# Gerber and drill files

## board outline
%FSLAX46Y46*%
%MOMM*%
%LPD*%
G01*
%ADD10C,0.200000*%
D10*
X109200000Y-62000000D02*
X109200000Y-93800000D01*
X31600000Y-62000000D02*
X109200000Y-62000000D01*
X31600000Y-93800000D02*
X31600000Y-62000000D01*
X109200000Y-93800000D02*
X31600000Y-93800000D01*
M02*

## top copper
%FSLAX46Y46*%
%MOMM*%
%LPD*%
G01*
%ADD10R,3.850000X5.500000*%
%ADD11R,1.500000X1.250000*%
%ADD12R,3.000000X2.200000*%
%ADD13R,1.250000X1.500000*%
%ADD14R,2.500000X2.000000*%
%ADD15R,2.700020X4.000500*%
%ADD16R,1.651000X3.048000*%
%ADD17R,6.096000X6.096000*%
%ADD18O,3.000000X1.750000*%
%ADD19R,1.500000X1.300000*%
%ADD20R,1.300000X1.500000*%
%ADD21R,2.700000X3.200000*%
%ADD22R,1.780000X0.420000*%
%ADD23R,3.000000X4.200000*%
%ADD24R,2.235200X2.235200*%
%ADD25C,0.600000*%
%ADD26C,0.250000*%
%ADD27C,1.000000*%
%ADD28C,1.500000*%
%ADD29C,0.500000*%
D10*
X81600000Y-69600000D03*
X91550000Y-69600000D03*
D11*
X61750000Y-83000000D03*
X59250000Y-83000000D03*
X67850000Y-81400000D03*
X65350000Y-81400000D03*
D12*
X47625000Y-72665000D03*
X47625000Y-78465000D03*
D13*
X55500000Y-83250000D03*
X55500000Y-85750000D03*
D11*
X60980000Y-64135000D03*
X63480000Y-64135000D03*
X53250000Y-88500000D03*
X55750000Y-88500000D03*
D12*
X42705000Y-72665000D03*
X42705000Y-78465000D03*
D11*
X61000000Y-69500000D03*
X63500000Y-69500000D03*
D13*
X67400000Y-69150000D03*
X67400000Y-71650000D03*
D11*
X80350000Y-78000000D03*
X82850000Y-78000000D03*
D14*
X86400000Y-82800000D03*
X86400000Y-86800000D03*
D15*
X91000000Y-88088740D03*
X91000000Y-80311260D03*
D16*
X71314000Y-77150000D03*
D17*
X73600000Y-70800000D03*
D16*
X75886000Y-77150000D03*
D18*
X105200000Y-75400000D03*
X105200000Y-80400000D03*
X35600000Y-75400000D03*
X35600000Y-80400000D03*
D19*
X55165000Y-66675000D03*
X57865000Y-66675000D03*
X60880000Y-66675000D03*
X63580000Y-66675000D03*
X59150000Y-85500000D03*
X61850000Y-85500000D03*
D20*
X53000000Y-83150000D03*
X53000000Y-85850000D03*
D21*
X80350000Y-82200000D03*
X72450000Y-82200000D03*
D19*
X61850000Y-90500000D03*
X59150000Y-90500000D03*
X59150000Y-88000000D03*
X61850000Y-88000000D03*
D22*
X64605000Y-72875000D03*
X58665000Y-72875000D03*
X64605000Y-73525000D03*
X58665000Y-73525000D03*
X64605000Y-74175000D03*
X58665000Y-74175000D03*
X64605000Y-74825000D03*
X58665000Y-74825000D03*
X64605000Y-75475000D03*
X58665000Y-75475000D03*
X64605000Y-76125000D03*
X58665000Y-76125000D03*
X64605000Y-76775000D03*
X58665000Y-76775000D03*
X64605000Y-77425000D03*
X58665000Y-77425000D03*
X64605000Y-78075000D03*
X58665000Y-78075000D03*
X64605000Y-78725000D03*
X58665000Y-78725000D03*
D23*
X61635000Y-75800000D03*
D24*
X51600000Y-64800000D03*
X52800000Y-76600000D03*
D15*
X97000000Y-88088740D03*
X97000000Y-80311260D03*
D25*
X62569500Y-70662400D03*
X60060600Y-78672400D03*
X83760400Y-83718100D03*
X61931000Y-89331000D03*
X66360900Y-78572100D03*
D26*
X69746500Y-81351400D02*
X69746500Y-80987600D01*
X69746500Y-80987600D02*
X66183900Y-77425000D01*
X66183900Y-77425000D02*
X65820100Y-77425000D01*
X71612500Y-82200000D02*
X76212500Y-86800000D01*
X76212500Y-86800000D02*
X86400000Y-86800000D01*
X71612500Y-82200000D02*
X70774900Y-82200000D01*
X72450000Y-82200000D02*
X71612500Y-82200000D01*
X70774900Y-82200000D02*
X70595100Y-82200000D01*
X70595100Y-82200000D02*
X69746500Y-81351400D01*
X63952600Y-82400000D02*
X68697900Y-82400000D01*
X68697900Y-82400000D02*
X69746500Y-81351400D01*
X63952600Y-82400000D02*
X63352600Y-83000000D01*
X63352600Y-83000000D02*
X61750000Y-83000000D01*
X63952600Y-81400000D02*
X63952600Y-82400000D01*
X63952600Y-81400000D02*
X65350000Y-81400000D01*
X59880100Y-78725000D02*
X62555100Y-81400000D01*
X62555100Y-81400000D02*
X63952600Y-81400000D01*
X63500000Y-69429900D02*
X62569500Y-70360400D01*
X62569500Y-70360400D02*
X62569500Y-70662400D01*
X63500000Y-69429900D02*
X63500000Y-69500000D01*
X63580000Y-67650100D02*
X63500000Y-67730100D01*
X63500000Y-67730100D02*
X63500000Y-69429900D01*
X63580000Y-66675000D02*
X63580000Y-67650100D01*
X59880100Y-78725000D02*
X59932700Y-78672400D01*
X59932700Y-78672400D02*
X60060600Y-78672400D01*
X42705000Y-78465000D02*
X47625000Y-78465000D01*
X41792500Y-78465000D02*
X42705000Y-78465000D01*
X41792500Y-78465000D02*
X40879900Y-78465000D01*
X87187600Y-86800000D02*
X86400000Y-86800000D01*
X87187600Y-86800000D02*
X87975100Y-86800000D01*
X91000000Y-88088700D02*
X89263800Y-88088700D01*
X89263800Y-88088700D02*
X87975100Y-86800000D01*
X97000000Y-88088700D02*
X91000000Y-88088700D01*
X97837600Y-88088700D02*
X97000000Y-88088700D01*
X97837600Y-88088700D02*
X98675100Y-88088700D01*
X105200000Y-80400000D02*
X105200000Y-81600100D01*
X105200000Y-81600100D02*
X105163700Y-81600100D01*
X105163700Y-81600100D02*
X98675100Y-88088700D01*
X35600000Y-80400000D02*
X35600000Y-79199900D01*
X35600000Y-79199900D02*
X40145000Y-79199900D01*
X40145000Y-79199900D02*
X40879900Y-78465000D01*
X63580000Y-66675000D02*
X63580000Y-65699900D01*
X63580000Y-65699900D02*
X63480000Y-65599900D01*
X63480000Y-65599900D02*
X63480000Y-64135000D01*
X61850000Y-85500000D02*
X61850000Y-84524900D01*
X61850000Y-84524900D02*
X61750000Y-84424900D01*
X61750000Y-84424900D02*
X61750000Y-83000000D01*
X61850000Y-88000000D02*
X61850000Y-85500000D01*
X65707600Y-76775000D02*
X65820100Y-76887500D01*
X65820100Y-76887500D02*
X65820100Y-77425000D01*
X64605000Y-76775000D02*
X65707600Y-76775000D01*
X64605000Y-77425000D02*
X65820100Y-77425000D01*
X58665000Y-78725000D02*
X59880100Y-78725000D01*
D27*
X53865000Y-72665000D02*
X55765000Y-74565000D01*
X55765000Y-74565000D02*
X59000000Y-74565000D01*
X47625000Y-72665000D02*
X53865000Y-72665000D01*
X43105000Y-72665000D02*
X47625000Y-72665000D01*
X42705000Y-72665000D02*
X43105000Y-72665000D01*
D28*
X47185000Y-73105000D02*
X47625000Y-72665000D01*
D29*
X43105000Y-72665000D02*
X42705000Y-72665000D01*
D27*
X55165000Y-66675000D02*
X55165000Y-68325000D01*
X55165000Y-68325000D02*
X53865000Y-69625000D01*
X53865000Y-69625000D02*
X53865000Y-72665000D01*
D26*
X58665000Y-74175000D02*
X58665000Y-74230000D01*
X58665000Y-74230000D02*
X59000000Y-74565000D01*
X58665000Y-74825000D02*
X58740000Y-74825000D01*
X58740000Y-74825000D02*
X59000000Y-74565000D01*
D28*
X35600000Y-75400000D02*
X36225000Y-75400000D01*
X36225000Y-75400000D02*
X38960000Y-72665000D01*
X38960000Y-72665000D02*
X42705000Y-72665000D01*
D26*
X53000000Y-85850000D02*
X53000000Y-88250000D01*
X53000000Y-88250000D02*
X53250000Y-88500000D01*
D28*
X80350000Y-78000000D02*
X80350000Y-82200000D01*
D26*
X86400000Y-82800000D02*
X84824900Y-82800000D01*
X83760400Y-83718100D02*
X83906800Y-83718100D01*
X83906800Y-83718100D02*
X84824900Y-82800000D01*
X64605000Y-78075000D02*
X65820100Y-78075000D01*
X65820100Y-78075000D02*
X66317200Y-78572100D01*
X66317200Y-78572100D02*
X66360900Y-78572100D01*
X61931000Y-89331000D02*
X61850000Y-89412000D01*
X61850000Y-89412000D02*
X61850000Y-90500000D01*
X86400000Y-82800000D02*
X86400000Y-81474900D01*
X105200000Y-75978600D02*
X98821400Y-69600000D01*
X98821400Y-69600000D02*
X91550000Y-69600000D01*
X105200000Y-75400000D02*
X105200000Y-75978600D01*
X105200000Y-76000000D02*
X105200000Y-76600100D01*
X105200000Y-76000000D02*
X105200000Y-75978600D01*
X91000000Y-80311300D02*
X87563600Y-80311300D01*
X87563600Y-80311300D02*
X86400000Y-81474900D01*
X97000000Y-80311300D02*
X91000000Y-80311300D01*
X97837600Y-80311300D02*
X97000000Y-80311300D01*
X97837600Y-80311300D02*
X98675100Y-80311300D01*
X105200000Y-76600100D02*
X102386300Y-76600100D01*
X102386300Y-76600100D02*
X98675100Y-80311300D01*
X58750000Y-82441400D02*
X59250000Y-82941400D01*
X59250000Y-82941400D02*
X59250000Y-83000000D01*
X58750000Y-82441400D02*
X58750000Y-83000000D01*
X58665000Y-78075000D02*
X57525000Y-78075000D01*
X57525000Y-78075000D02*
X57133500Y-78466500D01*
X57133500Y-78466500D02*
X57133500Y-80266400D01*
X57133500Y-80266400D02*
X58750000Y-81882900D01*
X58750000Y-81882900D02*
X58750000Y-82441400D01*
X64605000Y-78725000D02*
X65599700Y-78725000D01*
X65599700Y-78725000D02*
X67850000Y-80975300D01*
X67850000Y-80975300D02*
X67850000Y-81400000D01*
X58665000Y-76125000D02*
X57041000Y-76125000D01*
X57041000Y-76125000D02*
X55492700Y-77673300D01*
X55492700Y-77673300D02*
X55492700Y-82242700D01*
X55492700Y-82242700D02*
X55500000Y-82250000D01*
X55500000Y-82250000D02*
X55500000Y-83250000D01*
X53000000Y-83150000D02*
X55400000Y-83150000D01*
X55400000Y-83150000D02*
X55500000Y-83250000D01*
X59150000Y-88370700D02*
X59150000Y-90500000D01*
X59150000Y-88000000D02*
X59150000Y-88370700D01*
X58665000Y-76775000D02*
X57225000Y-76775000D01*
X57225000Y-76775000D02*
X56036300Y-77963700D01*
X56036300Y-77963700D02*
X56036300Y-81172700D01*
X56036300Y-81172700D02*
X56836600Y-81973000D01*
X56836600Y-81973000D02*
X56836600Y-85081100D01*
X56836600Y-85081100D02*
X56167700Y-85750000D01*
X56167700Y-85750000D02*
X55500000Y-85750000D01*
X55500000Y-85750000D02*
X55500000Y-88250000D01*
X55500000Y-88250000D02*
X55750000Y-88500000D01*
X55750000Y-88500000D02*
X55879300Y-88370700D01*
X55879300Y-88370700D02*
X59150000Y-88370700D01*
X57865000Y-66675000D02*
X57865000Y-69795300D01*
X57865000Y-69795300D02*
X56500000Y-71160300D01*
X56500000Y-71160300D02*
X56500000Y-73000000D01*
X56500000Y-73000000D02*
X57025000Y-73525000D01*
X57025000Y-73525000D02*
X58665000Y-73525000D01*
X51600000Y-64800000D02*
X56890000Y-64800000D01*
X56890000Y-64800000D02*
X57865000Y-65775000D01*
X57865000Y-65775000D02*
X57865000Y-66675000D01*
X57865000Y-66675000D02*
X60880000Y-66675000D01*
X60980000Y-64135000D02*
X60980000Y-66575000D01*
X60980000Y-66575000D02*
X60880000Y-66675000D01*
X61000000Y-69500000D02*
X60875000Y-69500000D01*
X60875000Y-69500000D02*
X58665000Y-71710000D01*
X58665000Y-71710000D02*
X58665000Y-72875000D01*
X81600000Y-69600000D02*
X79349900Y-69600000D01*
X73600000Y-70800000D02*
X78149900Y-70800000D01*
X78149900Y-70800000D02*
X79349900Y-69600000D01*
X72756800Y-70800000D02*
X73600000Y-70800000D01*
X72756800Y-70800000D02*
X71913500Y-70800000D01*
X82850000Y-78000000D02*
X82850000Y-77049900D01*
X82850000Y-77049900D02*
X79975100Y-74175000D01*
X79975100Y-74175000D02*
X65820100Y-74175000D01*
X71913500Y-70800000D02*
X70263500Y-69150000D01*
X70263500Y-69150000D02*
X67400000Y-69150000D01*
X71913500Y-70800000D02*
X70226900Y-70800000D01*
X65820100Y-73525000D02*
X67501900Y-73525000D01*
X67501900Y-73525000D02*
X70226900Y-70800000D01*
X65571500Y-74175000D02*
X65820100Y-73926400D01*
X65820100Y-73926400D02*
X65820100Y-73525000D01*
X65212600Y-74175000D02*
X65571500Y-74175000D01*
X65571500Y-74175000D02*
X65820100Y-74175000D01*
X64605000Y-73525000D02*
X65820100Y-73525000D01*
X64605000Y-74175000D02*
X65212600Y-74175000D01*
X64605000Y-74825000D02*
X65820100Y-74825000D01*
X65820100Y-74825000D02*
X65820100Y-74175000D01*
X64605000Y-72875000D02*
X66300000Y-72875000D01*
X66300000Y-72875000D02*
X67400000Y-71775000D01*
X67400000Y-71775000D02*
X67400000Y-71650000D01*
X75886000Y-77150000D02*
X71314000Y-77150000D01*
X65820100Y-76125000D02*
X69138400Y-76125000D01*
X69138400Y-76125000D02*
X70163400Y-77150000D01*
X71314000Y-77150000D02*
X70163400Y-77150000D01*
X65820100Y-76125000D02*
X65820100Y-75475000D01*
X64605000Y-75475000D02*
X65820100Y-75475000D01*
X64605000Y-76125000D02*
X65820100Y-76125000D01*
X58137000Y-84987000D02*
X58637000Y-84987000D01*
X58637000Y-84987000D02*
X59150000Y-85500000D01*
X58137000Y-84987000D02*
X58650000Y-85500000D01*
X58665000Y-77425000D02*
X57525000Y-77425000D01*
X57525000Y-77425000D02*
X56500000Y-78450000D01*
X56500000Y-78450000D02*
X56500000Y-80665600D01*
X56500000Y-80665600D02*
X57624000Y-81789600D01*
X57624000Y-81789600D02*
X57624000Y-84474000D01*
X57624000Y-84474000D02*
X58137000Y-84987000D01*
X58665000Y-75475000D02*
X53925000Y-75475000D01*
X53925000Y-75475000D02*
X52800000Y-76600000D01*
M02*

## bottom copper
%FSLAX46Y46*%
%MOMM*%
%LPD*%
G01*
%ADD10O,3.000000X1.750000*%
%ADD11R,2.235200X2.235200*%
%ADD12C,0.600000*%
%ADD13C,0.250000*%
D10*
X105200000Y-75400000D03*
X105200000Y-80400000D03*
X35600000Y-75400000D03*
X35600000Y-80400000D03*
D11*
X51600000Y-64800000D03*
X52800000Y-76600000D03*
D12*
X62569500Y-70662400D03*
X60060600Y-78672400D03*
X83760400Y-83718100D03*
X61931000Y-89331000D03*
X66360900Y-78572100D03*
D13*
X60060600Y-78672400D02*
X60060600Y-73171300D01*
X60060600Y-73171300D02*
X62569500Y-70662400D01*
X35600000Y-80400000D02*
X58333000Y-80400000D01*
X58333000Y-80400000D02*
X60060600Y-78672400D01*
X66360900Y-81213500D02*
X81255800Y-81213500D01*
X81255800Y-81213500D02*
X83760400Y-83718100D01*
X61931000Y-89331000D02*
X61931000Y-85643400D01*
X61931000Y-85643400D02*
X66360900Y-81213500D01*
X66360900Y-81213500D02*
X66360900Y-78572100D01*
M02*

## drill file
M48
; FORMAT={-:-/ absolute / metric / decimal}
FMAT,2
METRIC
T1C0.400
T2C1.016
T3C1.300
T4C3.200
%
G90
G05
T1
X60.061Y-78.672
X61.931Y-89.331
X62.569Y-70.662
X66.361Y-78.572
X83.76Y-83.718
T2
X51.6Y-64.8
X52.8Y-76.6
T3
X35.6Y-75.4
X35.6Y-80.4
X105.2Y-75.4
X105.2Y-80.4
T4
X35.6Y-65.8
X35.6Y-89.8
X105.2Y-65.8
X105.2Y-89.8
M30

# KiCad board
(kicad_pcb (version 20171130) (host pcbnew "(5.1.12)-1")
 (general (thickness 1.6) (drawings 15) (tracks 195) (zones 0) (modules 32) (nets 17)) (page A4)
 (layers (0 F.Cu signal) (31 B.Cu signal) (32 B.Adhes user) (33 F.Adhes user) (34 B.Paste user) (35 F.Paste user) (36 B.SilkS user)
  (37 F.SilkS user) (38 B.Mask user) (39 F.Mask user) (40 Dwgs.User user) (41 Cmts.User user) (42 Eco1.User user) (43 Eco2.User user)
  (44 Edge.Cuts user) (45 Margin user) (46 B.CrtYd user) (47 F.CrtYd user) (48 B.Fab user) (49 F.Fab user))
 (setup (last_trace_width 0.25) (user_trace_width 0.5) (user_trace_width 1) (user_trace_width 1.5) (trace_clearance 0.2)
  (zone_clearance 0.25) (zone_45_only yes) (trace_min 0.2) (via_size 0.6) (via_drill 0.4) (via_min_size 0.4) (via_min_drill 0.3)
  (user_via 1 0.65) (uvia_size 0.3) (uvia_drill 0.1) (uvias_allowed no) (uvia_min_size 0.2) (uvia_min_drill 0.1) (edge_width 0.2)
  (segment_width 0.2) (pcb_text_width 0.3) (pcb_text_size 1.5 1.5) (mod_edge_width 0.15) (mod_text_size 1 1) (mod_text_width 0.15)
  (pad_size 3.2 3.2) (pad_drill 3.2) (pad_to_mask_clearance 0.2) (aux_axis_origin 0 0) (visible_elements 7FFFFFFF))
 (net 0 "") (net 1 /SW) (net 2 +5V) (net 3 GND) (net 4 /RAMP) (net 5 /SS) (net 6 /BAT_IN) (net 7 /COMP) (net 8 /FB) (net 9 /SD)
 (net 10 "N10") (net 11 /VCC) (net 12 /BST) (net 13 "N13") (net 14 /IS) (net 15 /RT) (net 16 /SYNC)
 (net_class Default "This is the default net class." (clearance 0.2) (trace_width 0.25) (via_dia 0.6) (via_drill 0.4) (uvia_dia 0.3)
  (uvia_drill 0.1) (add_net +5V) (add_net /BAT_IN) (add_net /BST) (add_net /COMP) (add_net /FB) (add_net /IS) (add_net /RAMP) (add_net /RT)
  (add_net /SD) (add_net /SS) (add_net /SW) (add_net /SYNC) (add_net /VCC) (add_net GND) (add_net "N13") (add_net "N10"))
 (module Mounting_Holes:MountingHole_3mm (layer F.Cu) (at 35.6 89.8)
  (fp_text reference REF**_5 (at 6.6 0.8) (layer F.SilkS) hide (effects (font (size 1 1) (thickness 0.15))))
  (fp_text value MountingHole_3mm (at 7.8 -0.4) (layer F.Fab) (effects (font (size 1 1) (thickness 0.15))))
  (pad "" np_thru_hole circle (at 0 0) (size 3.2 3.2) (drill 3.2) (layers *.Cu *.Mask F.SilkS)))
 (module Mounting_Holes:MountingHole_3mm (layer F.Cu) (at 35.6 65.8)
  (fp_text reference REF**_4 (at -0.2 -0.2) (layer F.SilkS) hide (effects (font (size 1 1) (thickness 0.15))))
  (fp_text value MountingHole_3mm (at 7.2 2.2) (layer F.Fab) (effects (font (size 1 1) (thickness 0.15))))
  (pad "" np_thru_hole circle (at 0 0) (size 3.2 3.2) (drill 3.2) (layers *.Cu *.Mask F.SilkS)))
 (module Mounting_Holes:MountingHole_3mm (layer F.Cu) (at 105.2 89.8)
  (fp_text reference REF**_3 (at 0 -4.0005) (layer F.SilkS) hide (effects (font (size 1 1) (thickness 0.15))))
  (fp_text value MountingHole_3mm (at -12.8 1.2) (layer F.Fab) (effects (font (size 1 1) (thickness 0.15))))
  (pad "" np_thru_hole circle (at 0 0) (size 3.2 3.2) (drill 3.2) (layers *.Cu *.Mask F.SilkS)))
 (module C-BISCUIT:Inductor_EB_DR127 (layer F.Cu) (at 81.6 69.6)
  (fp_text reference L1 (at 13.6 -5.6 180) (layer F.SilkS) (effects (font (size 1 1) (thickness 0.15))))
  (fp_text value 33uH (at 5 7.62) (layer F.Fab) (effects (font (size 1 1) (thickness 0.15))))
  (pad 1 smd rect (at 0 0) (size 3.85 5.5) (layers F.Cu F.Paste F.Mask) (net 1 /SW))
  (pad 2 smd rect (at 9.95 0) (size 3.85 5.5) (layers F.Cu F.Paste F.Mask) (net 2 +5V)))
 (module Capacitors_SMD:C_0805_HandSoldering (layer F.Cu) (at 60.5 83 180)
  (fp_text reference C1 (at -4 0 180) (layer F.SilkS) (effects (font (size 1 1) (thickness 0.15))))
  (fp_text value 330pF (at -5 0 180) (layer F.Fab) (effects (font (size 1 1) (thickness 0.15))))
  (pad 1 smd rect (at -1.25 0 180) (size 1.5 1.25) (layers F.Cu F.Paste F.Mask) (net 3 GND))
  (pad 2 smd rect (at 1.25 0 180) (size 1.5 1.25) (layers F.Cu F.Paste F.Mask) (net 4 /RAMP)))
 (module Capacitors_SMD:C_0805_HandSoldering (layer F.Cu) (at 66.6 81.4 180)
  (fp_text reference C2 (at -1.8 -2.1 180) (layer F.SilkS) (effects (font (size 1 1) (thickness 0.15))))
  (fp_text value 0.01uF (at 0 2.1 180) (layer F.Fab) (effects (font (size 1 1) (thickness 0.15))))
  (pad 1 smd rect (at -1.25 0 180) (size 1.5 1.25) (layers F.Cu F.Paste F.Mask) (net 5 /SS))
  (pad 2 smd rect (at 1.25 0 180) (size 1.5 1.25) (layers F.Cu F.Paste F.Mask) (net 3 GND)))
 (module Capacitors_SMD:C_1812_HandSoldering (layer F.Cu) (at 47.625 75.565 270)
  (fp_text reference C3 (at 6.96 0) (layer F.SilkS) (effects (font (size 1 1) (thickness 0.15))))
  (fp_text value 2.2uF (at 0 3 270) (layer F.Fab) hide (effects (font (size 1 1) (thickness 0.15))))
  (pad 1 smd rect (at -2.9 0 270) (size 2.2 3) (layers F.Cu F.Paste F.Mask) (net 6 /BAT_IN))
  (pad 2 smd rect (at 2.9 0 270) (size 2.2 3) (layers F.Cu F.Paste F.Mask) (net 3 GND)))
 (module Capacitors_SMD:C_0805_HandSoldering (layer F.Cu) (at 55.5 84.5 270)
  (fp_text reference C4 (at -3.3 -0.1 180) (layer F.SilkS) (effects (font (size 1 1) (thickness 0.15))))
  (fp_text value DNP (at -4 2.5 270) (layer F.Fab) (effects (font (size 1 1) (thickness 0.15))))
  (pad 1 smd rect (at -1.25 0 270) (size 1.5 1.25) (layers F.Cu F.Paste F.Mask) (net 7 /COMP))
  (pad 2 smd rect (at 1.25 0 270) (size 1.5 1.25) (layers F.Cu F.Paste F.Mask) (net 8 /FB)))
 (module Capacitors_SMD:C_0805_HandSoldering (layer F.Cu) (at 62.23 64.135)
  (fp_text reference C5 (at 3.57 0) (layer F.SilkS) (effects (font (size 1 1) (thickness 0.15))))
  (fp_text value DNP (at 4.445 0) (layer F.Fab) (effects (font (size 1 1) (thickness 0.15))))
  (pad 1 smd rect (at -1.25 0) (size 1.5 1.25) (layers F.Cu F.Paste F.Mask) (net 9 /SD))
  (pad 2 smd rect (at 1.25 0) (size 1.5 1.25) (layers F.Cu F.Paste F.Mask) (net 3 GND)))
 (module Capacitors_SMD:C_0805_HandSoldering (layer F.Cu) (at 54.5 88.5)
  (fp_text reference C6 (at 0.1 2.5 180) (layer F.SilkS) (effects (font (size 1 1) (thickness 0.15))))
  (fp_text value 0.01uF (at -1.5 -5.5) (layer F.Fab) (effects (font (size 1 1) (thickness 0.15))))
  (pad 1 smd rect (at -1.25 0) (size 1.5 1.25) (layers F.Cu F.Paste F.Mask) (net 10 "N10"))
  (pad 2 smd rect (at 1.25 0) (size 1.5 1.25) (layers F.Cu F.Paste F.Mask) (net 8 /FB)))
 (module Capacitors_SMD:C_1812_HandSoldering (layer F.Cu) (at 42.705 75.565 270)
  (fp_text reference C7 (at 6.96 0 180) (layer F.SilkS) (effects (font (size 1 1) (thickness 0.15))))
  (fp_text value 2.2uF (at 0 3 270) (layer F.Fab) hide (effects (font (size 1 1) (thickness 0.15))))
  (pad 1 smd rect (at -2.9 0 270) (size 2.2 3) (layers F.Cu F.Paste F.Mask) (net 6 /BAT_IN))
  (pad 2 smd rect (at 2.9 0 270) (size 2.2 3) (layers F.Cu F.Paste F.Mask) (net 3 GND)))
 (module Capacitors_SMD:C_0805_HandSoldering (layer F.Cu) (at 62.25 69.5)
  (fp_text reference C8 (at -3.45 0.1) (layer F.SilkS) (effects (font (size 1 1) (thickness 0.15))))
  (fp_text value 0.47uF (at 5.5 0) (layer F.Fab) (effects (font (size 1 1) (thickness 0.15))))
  (pad 1 smd rect (at -1.25 0) (size 1.5 1.25) (layers F.Cu F.Paste F.Mask) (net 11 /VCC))
  (pad 2 smd rect (at 1.25 0) (size 1.5 1.25) (layers F.Cu F.Paste F.Mask) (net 3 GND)))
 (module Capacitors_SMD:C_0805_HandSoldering (layer F.Cu) (at 67.4 70.4 270)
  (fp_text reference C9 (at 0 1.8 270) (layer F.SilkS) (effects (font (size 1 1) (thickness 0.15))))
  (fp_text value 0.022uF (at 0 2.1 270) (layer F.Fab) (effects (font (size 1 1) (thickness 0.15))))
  (pad 1 smd rect (at -1.25 0 270) (size 1.5 1.25) (layers F.Cu F.Paste F.Mask) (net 1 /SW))
  (pad 2 smd rect (at 1.25 0 270) (size 1.5 1.25) (layers F.Cu F.Paste F.Mask) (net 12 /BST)))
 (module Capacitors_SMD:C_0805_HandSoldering (layer F.Cu) (at 81.6 78)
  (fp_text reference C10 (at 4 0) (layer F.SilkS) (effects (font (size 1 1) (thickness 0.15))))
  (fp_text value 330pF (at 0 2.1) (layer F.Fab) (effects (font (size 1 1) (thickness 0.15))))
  (pad 1 smd rect (at -1.25 0) (size 1.5 1.25) (layers F.Cu F.Paste F.Mask) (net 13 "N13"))
  (pad 2 smd rect (at 1.25 0) (size 1.5 1.25) (layers F.Cu F.Paste F.Mask) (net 1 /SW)))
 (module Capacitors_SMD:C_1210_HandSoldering (layer F.Cu) (at 86.4 84.8 270)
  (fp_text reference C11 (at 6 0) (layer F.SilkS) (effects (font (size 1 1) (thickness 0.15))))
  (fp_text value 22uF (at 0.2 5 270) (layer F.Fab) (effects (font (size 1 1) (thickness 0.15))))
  (pad 1 smd rect (at -2 0 270) (size 2 2.5) (layers F.Cu F.Paste F.Mask) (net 2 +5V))
  (pad 2 smd rect (at 2 0 270) (size 2 2.5) (layers F.Cu F.Paste F.Mask) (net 3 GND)))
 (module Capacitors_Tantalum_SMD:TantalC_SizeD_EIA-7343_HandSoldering (layer F.Cu) (at 91 84.2 270)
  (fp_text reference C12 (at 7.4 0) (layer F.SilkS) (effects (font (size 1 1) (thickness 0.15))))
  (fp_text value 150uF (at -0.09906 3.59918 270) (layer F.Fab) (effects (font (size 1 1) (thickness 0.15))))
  (pad 2 smd rect (at 3.88874 0 270) (size 4.0005 2.70002) (layers F.Cu F.Paste F.Mask) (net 3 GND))
  (pad 1 smd rect (at -3.88874 0 270) (size 4.0005 2.70002) (layers F.Cu F.Paste F.Mask) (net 2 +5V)))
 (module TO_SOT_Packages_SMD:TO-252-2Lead (layer F.Cu) (at 73.6 77.15)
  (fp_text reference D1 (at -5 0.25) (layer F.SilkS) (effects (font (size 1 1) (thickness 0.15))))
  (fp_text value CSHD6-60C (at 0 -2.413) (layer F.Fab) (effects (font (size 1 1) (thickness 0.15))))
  (pad 1 smd rect (at -2.286 0) (size 1.651 3.048) (layers F.Cu F.Paste F.Mask) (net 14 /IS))
  (pad 2 smd rect (at 0 -6.35) (size 6.096 6.096) (layers F.Cu F.Paste F.Mask) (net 1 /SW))
  (pad 3 smd rect (at 2.286 0) (size 1.651 3.048) (layers F.Cu F.Paste F.Mask) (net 14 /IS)))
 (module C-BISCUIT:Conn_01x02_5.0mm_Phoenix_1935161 (layer F.Cu) (at 105.2 75.4 270)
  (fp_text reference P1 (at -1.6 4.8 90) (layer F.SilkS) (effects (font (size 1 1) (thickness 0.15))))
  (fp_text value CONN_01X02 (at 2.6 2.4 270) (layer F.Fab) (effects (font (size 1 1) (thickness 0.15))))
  (pad 1 thru_hole oval (at 0 0 270) (size 1.75 3) (drill 1.3) (layers *.Cu *.Mask) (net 2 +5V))
  (pad 2 thru_hole oval (at 5 0 270) (size 1.75 3) (drill 1.3) (layers *.Cu *.Mask) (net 3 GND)))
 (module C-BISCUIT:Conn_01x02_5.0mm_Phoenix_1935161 (layer F.Cu) (at 35.6 75.4 270)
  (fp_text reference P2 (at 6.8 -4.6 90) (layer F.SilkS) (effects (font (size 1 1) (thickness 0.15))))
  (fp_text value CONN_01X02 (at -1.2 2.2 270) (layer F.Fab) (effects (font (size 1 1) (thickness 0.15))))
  (pad 1 thru_hole oval (at 0 0 270) (size 1.75 3) (drill 1.3) (layers *.Cu *.Mask) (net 6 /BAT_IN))
  (pad 2 thru_hole oval (at 5 0 270) (size 1.75 3) (drill 1.3) (layers *.Cu *.Mask) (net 3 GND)))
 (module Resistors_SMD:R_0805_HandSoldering (layer F.Cu) (at 56.515 66.675)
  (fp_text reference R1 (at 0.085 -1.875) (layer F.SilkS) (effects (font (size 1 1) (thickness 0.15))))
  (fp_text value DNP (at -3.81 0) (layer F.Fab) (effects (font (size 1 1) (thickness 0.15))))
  (pad 1 smd rect (at -1.35 0) (size 1.5 1.3) (layers F.Cu F.Paste F.Mask) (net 6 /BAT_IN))
  (pad 2 smd rect (at 1.35 0) (size 1.5 1.3) (layers F.Cu F.Paste F.Mask) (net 9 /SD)))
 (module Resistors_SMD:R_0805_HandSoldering (layer F.Cu) (at 62.23 66.675)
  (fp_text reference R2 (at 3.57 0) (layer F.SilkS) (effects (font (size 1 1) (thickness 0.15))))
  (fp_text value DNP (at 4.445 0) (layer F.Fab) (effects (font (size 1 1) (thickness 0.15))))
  (pad 1 smd rect (at -1.35 0) (size 1.5 1.3) (layers F.Cu F.Paste F.Mask) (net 9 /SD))
  (pad 2 smd rect (at 1.35 0) (size 1.5 1.3) (layers F.Cu F.Paste F.Mask) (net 3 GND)))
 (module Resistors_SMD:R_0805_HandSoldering (layer F.Cu) (at 60.5 85.5)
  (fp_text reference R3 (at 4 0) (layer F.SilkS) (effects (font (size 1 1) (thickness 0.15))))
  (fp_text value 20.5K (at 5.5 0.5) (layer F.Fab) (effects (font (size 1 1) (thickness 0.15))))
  (pad 1 smd rect (at -1.35 0) (size 1.5 1.3) (layers F.Cu F.Paste F.Mask) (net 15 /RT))
  (pad 2 smd rect (at 1.35 0) (size 1.5 1.3) (layers F.Cu F.Paste F.Mask) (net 3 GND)))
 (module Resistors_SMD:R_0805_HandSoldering (layer F.Cu) (at 53 84.5 270)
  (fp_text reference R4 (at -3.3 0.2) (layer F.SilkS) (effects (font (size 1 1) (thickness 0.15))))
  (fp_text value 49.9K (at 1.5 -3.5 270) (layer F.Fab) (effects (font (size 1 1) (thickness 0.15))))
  (pad 1 smd rect (at -1.35 0 270) (size 1.5 1.3) (layers F.Cu F.Paste F.Mask) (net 7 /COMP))
  (pad 2 smd rect (at 1.35 0 270) (size 1.5 1.3) (layers F.Cu F.Paste F.Mask) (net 10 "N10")))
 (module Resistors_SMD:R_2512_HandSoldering (layer F.Cu) (at 76.4 82.2 180)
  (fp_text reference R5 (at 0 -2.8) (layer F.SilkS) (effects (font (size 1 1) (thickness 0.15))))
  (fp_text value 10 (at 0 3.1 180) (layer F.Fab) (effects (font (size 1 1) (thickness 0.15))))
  (pad 1 smd rect (at -3.95 0 180) (size 2.7 3.2) (layers F.Cu F.Paste F.Mask) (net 13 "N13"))
  (pad 2 smd rect (at 3.95 0 180) (size 2.7 3.2) (layers F.Cu F.Paste F.Mask) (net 3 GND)))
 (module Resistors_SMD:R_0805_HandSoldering (layer F.Cu) (at 60.5 90.5 180)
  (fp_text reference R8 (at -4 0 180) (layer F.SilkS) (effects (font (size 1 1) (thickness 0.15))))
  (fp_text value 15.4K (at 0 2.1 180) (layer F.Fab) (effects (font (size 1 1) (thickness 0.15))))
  (pad 1 smd rect (at -1.35 0 180) (size 1.5 1.3) (layers F.Cu F.Paste F.Mask) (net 2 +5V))
  (pad 2 smd rect (at 1.35 0 180) (size 1.5 1.3) (layers F.Cu F.Paste F.Mask) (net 8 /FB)))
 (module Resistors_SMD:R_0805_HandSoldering (layer F.Cu) (at 60.5 88)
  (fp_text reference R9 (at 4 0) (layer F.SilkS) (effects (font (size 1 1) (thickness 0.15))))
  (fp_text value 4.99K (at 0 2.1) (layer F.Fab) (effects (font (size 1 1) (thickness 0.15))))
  (pad 1 smd rect (at -1.35 0) (size 1.5 1.3) (layers F.Cu F.Paste F.Mask) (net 8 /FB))
  (pad 2 smd rect (at 1.35 0) (size 1.5 1.3) (layers F.Cu F.Paste F.Mask) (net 3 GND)))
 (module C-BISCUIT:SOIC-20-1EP (layer F.Cu) (at 61.635 75.8 270)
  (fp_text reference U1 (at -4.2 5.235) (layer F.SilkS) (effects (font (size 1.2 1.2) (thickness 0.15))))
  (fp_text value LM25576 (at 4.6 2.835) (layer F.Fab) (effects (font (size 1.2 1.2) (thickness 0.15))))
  (pad 20 smd rect (at -2.925 -2.97 270) (size 0.42 1.78) (layers F.Cu F.Paste F.Mask) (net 12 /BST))
  (pad 1 smd rect (at -2.925 2.97 270) (size 0.42 1.78) (layers F.Cu F.Paste F.Mask) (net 11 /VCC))
  (pad 19 smd rect (at -2.275 -2.97 270) (size 0.42 1.78) (layers F.Cu F.Paste F.Mask) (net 1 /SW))
  (pad 2 smd rect (at -2.275 2.97 270) (size 0.42 1.78) (layers F.Cu F.Paste F.Mask) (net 9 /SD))
  (pad 18 smd rect (at -1.625 -2.97 270) (size 0.42 1.78) (layers F.Cu F.Paste F.Mask) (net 1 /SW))
  (pad 3 smd rect (at -1.625 2.97 270) (size 0.42 1.78) (layers F.Cu F.Paste F.Mask) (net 6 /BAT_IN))
  (pad 17 smd rect (at -0.975 -2.97 270) (size 0.42 1.78) (layers F.Cu F.Paste F.Mask) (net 1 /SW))
  (pad 4 smd rect (at -0.975 2.97 270) (size 0.42 1.78) (layers F.Cu F.Paste F.Mask) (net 6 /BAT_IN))
  (pad 16 smd rect (at -0.325 -2.97 270) (size 0.42 1.78) (layers F.Cu F.Paste F.Mask) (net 14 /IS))
  (pad 5 smd rect (at -0.325 2.97 270) (size 0.42 1.78) (layers F.Cu F.Paste F.Mask) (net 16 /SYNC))
  (pad 15 smd rect (at 0.325 -2.97 270) (size 0.42 1.78) (layers F.Cu F.Paste F.Mask) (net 14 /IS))
  (pad 6 smd rect (at 0.325 2.97 270) (size 0.42 1.78) (layers F.Cu F.Paste F.Mask) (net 7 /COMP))
  (pad 14 smd rect (at 0.975 -2.97 270) (size 0.42 1.78) (layers F.Cu F.Paste F.Mask) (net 3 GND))
  (pad 7 smd rect (at 0.975 2.97 270) (size 0.42 1.78) (layers F.Cu F.Paste F.Mask) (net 8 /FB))
  (pad 13 smd rect (at 1.625 -2.97 270) (size 0.42 1.78) (layers F.Cu F.Paste F.Mask) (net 3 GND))
  (pad 8 smd rect (at 1.625 2.97 270) (size 0.42 1.78) (layers F.Cu F.Paste F.Mask) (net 15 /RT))
  (pad 12 smd rect (at 2.275 -2.97 270) (size 0.42 1.78) (layers F.Cu F.Paste F.Mask) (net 2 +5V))
  (pad 9 smd rect (at 2.275 2.97 270) (size 0.42 1.78) (layers F.Cu F.Paste F.Mask) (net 4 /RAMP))
  (pad 11 smd rect (at 2.925 -2.97 270) (size 0.42 1.78) (layers F.Cu F.Paste F.Mask) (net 5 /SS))
  (pad 10 smd rect (at 2.925 2.97 270) (size 0.42 1.78) (layers F.Cu F.Paste F.Mask) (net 3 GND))
  (pad EP smd rect (at 0 0 270) (size 4.2 3) (layers F.Cu F.Paste F.Mask)))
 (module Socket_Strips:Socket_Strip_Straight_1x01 (layer F.Cu) (at 51.6 64.8)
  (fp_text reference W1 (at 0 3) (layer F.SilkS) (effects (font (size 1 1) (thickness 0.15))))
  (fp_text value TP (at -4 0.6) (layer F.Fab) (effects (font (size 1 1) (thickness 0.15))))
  (pad 1 thru_hole rect (at 0 0) (size 2.2352 2.2352) (drill 1.016) (layers *.Cu *.Mask F.SilkS) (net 9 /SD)))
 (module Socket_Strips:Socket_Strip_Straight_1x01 (layer F.Cu) (at 52.8 76.6)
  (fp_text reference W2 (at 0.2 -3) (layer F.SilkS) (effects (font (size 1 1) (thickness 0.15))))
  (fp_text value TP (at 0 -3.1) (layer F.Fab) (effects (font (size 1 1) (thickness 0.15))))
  (pad 1 thru_hole rect (at 0 0) (size 2.2352 2.2352) (drill 1.016) (layers *.Cu *.Mask F.SilkS) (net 16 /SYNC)))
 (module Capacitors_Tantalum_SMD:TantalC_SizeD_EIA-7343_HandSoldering (layer F.Cu) (at 97 84.2 270)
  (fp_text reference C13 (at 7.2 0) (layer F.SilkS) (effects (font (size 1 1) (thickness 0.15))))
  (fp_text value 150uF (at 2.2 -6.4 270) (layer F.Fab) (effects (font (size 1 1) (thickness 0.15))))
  (pad 2 smd rect (at 3.88874 0 270) (size 4.0005 2.70002) (layers F.Cu F.Paste F.Mask) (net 3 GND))
  (pad 1 smd rect (at -3.88874 0 270) (size 4.0005 2.70002) (layers F.Cu F.Paste F.Mask) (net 2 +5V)))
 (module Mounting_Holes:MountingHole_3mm (layer F.Cu) (at 105.2 65.8)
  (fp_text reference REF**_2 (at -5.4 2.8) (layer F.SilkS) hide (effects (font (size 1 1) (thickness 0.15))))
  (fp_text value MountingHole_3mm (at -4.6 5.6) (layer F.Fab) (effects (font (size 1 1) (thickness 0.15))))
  (pad "" np_thru_hole circle (at 0 0) (size 3.2 3.2) (drill 3.2) (layers *.Cu *.Mask F.SilkS)))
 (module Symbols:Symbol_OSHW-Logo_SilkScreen (layer F.Cu) (at 45 65.8)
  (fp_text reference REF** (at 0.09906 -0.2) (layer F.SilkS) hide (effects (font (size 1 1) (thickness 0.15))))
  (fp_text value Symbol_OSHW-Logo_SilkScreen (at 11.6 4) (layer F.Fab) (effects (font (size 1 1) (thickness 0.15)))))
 (gr_line (start 109.2 62) (end 109.2 93.8) (layer Edge.Cuts) (width 0.2))
 (gr_line (start 31.6 62) (end 109.2 62) (layer Edge.Cuts) (width 0.2))
 (gr_line (start 31.6 93.8) (end 31.6 62) (layer Edge.Cuts) (width 0.2))
 (gr_line (start 109.2 93.8) (end 31.6 93.8) (layer Edge.Cuts) (width 0.2))
 (segment (start 69.7465 81.3514) (end 69.7465 80.9876) (width 0.25) (layer F.Cu) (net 3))
 (segment (start 69.7465 80.9876) (end 66.1839 77.425) (width 0.25) (layer F.Cu) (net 3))
 (segment (start 66.1839 77.425) (end 65.8201 77.425) (width 0.25) (layer F.Cu) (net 3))
 (segment (start 71.6125 82.2) (end 76.2125 86.8) (width 0.25) (layer F.Cu) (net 3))
 (segment (start 76.2125 86.8) (end 86.4 86.8) (width 0.25) (layer F.Cu) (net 3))
 (segment (start 71.6125 82.2) (end 70.7749 82.2) (width 0.25) (layer F.Cu) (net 3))
 (segment (start 72.45 82.2) (end 71.6125 82.2) (width 0.25) (layer F.Cu) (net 3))
 (segment (start 70.7749 82.2) (end 70.5951 82.2) (width 0.25) (layer F.Cu) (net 3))
 (segment (start 70.5951 82.2) (end 69.7465 81.3514) (width 0.25) (layer F.Cu) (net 3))
 (segment (start 63.9526 82.4) (end 68.6979 82.4) (width 0.25) (layer F.Cu) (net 3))
 (segment (start 68.6979 82.4) (end 69.7465 81.3514) (width 0.25) (layer F.Cu) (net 3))
 (segment (start 63.9526 82.4) (end 63.3526 83) (width 0.25) (layer F.Cu) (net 3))
 (segment (start 63.3526 83) (end 61.75 83) (width 0.25) (layer F.Cu) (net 3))
 (segment (start 63.9526 81.4) (end 63.9526 82.4) (width 0.25) (layer F.Cu) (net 3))
 (segment (start 63.9526 81.4) (end 65.35 81.4) (width 0.25) (layer F.Cu) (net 3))
 (segment (start 59.8801 78.725) (end 62.5551 81.4) (width 0.25) (layer F.Cu) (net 3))
 (segment (start 62.5551 81.4) (end 63.9526 81.4) (width 0.25) (layer F.Cu) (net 3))
 (segment (start 63.5 69.4299) (end 62.5695 70.3604) (width 0.25) (layer F.Cu) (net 3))
 (segment (start 62.5695 70.3604) (end 62.5695 70.6624) (width 0.25) (layer F.Cu) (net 3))
 (segment (start 60.0606 78.6724) (end 60.0606 73.1713) (width 0.25) (layer B.Cu) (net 3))
 (segment (start 60.0606 73.1713) (end 62.5695 70.6624) (width 0.25) (layer B.Cu) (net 3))
 (segment (start 63.5 69.4299) (end 63.5 69.5) (width 0.25) (layer F.Cu) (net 3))
 (segment (start 63.58 67.6501) (end 63.5 67.7301) (width 0.25) (layer F.Cu) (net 3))
 (segment (start 63.5 67.7301) (end 63.5 69.4299) (width 0.25) (layer F.Cu) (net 3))
 (segment (start 63.58 66.675) (end 63.58 67.6501) (width 0.25) (layer F.Cu) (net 3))
 (segment (start 59.8801 78.725) (end 59.9327 78.6724) (width 0.25) (layer F.Cu) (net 3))
 (segment (start 59.9327 78.6724) (end 60.0606 78.6724) (width 0.25) (layer F.Cu) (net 3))
 (segment (start 35.6 80.4) (end 58.333 80.4) (width 0.25) (layer B.Cu) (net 3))
 (segment (start 58.333 80.4) (end 60.0606 78.6724) (width 0.25) (layer B.Cu) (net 3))
 (segment (start 42.705 78.465) (end 47.625 78.465) (width 0.25) (layer F.Cu) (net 3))
 (segment (start 41.7925 78.465) (end 42.705 78.465) (width 0.25) (layer F.Cu) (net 3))
 (segment (start 41.7925 78.465) (end 40.8799 78.465) (width 0.25) (layer F.Cu) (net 3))
 (segment (start 87.1876 86.8) (end 86.4 86.8) (width 0.25) (layer F.Cu) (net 3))
 (segment (start 87.1876 86.8) (end 87.9751 86.8) (width 0.25) (layer F.Cu) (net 3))
 (segment (start 91 88.0887) (end 89.2638 88.0887) (width 0.25) (layer F.Cu) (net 3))
 (segment (start 89.2638 88.0887) (end 87.9751 86.8) (width 0.25) (layer F.Cu) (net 3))
 (segment (start 97 88.0887) (end 91 88.0887) (width 0.25) (layer F.Cu) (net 3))
 (segment (start 97.8376 88.0887) (end 97 88.0887) (width 0.25) (layer F.Cu) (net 3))
 (segment (start 97.8376 88.0887) (end 98.6751 88.0887) (width 0.25) (layer F.Cu) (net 3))
 (segment (start 105.2 80.4) (end 105.2 81.6001) (width 0.25) (layer F.Cu) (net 3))
 (segment (start 105.2 81.6001) (end 105.1637 81.6001) (width 0.25) (layer F.Cu) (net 3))
 (segment (start 105.1637 81.6001) (end 98.6751 88.0887) (width 0.25) (layer F.Cu) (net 3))
 (segment (start 35.6 80.4) (end 35.6 79.1999) (width 0.25) (layer F.Cu) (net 3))
 (segment (start 35.6 79.1999) (end 40.145 79.1999) (width 0.25) (layer F.Cu) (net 3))
 (segment (start 40.145 79.1999) (end 40.8799 78.465) (width 0.25) (layer F.Cu) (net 3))
 (segment (start 63.58 66.675) (end 63.58 65.6999) (width 0.25) (layer F.Cu) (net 3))
 (segment (start 63.58 65.6999) (end 63.48 65.5999) (width 0.25) (layer F.Cu) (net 3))
 (segment (start 63.48 65.5999) (end 63.48 64.135) (width 0.25) (layer F.Cu) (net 3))
 (segment (start 61.85 85.5) (end 61.85 84.5249) (width 0.25) (layer F.Cu) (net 3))
 (segment (start 61.85 84.5249) (end 61.75 84.4249) (width 0.25) (layer F.Cu) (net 3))
 (segment (start 61.75 84.4249) (end 61.75 83) (width 0.25) (layer F.Cu) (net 3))
 (segment (start 61.85 88) (end 61.85 85.5) (width 0.25) (layer F.Cu) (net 3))
 (segment (start 65.7076 76.775) (end 65.8201 76.8875) (width 0.25) (layer F.Cu) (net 3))
 (segment (start 65.8201 76.8875) (end 65.8201 77.425) (width 0.25) (layer F.Cu) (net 3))
 (segment (start 64.605 76.775) (end 65.7076 76.775) (width 0.25) (layer F.Cu) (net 3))
 (segment (start 64.605 77.425) (end 65.8201 77.425) (width 0.25) (layer F.Cu) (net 3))
 (segment (start 58.665 78.725) (end 59.8801 78.725) (width 0.25) (layer F.Cu) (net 3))
 (via (at 62.5695 70.6624) (size 0.6) (layers F.Cu B.Cu) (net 3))
 (via (at 60.0606 78.6724) (size 0.6) (layers F.Cu B.Cu) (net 3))
 (segment (start 53.865 72.665) (end 55.765 74.565) (width 1) (layer F.Cu) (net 6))
 (segment (start 55.765 74.565) (end 59 74.565) (width 1) (layer F.Cu) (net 6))
 (segment (start 47.625 72.665) (end 53.865 72.665) (width 1) (layer F.Cu) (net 6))
 (segment (start 43.105 72.665) (end 47.625 72.665) (width 1) (layer F.Cu) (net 6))
 (segment (start 42.705 72.665) (end 43.105 72.665) (width 1) (layer F.Cu) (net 6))
 (segment (start 47.185 73.105) (end 47.625 72.665) (width 1.5) (layer F.Cu) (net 6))
 (segment (start 43.105 72.665) (end 42.705 72.665) (width 0.5) (layer F.Cu) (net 6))
 (segment (start 55.165 66.675) (end 55.165 68.325) (width 1) (layer F.Cu) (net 6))
 (segment (start 55.165 68.325) (end 53.865 69.625) (width 1) (layer F.Cu) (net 6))
 (segment (start 53.865 69.625) (end 53.865 72.665) (width 1) (layer F.Cu) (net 6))
 (segment (start 58.665 74.175) (end 58.665 74.23) (width 0.25) (layer F.Cu) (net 6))
 (segment (start 58.665 74.23) (end 59 74.565) (width 0.25) (layer F.Cu) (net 6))
 (segment (start 58.665 74.825) (end 58.74 74.825) (width 0.25) (layer F.Cu) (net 6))
 (segment (start 58.74 74.825) (end 59 74.565) (width 0.25) (layer F.Cu) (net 6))
 (segment (start 35.6 75.4) (end 36.225 75.4) (width 1.5) (layer F.Cu) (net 6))
 (segment (start 36.225 75.4) (end 38.96 72.665) (width 1.5) (layer F.Cu) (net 6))
 (segment (start 38.96 72.665) (end 42.705 72.665) (width 1.5) (layer F.Cu) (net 6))
 (segment (start 53 85.85) (end 53 88.25) (width 0.25) (layer F.Cu) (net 10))
 (segment (start 53 88.25) (end 53.25 88.5) (width 0.25) (layer F.Cu) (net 10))
 (segment (start 80.35 78) (end 80.35 82.2) (width 1.5) (layer F.Cu) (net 13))
 (segment (start 66.3609 81.2135) (end 81.2558 81.2135) (width 0.25) (layer B.Cu) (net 2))
 (segment (start 81.2558 81.2135) (end 83.7604 83.7181) (width 0.25) (layer B.Cu) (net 2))
 (segment (start 61.931 89.331) (end 61.931 85.6434) (width 0.25) (layer B.Cu) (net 2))
 (segment (start 61.931 85.6434) (end 66.3609 81.2135) (width 0.25) (layer B.Cu) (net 2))
 (segment (start 66.3609 81.2135) (end 66.3609 78.5721) (width 0.25) (layer B.Cu) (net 2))
 (segment (start 86.4 82.8) (end 84.8249 82.8) (width 0.25) (layer F.Cu) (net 2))
 (segment (start 83.7604 83.7181) (end 83.9068 83.7181) (width 0.25) (layer F.Cu) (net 2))
 (segment (start 83.9068 83.7181) (end 84.8249 82.8) (width 0.25) (layer F.Cu) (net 2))
 (segment (start 64.605 78.075) (end 65.8201 78.075) (width 0.25) (layer F.Cu) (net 2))
 (segment (start 65.8201 78.075) (end 66.3172 78.5721) (width 0.25) (layer F.Cu) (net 2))
 (segment (start 66.3172 78.5721) (end 66.3609 78.5721) (width 0.25) (layer F.Cu) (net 2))
 (segment (start 61.931 89.331) (end 61.85 89.412) (width 0.25) (layer F.Cu) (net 2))
 (segment (start 61.85 89.412) (end 61.85 90.5) (width 0.25) (layer F.Cu) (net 2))
 (segment (start 86.4 82.8) (end 86.4 81.4749) (width 0.25) (layer F.Cu) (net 2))
 (segment (start 105.2 75.9786) (end 98.8214 69.6) (width 0.25) (layer F.Cu) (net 2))
 (segment (start 98.8214 69.6) (end 91.55 69.6) (width 0.25) (layer F.Cu) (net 2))
 (segment (start 105.2 75.4) (end 105.2 75.9786) (width 0.25) (layer F.Cu) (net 2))
 (segment (start 105.2 76) (end 105.2 76.6001) (width 0.25) (layer F.Cu) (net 2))
 (segment (start 105.2 76) (end 105.2 75.9786) (width 0.25) (layer F.Cu) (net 2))
 (segment (start 91 80.3113) (end 87.5636 80.3113) (width 0.25) (layer F.Cu) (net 2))
 (segment (start 87.5636 80.3113) (end 86.4 81.4749) (width 0.25) (layer F.Cu) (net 2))
 (segment (start 97 80.3113) (end 91 80.3113) (width 0.25) (layer F.Cu) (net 2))
 (segment (start 97.8376 80.3113) (end 97 80.3113) (width 0.25) (layer F.Cu) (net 2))
 (segment (start 97.8376 80.3113) (end 98.6751 80.3113) (width 0.25) (layer F.Cu) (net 2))
 (segment (start 105.2 76.6001) (end 102.3863 76.6001) (width 0.25) (layer F.Cu) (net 2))
 (segment (start 102.3863 76.6001) (end 98.6751 80.3113) (width 0.25) (layer F.Cu) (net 2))
 (via (at 83.7604 83.7181) (size 0.6) (layers F.Cu B.Cu) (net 2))
 (via (at 61.931 89.331) (size 0.6) (layers F.Cu B.Cu) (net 2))
 (via (at 66.3609 78.5721) (size 0.6) (layers F.Cu B.Cu) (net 2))
 (segment (start 58.75 82.4414) (end 59.25 82.9414) (width 0.25) (layer F.Cu) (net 4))
 (segment (start 59.25 82.9414) (end 59.25 83) (width 0.25) (layer F.Cu) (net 4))
 (segment (start 58.75 82.4414) (end 58.75 83) (width 0.25) (layer F.Cu) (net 4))
 (segment (start 58.665 78.075) (end 57.525 78.075) (width 0.25) (layer F.Cu) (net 4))
 (segment (start 57.525 78.075) (end 57.1335 78.4665) (width 0.25) (layer F.Cu) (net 4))
 (segment (start 57.1335 78.4665) (end 57.1335 80.2664) (width 0.25) (layer F.Cu) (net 4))
 (segment (start 57.1335 80.2664) (end 58.75 81.8829) (width 0.25) (layer F.Cu) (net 4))
 (segment (start 58.75 81.8829) (end 58.75 82.4414) (width 0.25) (layer F.Cu) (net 4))
 (segment (start 64.605 78.725) (end 65.5997 78.725) (width 0.25) (layer F.Cu) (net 5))
 (segment (start 65.5997 78.725) (end 67.85 80.9753) (width 0.25) (layer F.Cu) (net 5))
 (segment (start 67.85 80.9753) (end 67.85 81.4) (width 0.25) (layer F.Cu) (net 5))
 (segment (start 58.665 76.125) (end 57.041 76.125) (width 0.25) (layer F.Cu) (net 7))
 (segment (start 57.041 76.125) (end 55.4927 77.6733) (width 0.25) (layer F.Cu) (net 7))
 (segment (start 55.4927 77.6733) (end 55.4927 82.2427) (width 0.25) (layer F.Cu) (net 7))
 (segment (start 55.4927 82.2427) (end 55.5 82.25) (width 0.25) (layer F.Cu) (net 7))
 (segment (start 55.5 82.25) (end 55.5 83.25) (width 0.25) (layer F.Cu) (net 7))
 (segment (start 53 83.15) (end 55.4 83.15) (width 0.25) (layer F.Cu) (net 7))
 (segment (start 55.4 83.15) (end 55.5 83.25) (width 0.25) (layer F.Cu) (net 7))
 (segment (start 59.15 88.3707) (end 59.15 90.5) (width 0.25) (layer F.Cu) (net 8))
 (segment (start 59.15 88) (end 59.15 88.3707) (width 0.25) (layer F.Cu) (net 8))
 (segment (start 58.665 76.775) (end 57.225 76.775) (width 0.25) (layer F.Cu) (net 8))
 (segment (start 57.225 76.775) (end 56.0363 77.9637) (width 0.25) (layer F.Cu) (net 8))
 (segment (start 56.0363 77.9637) (end 56.0363 81.1727) (width 0.25) (layer F.Cu) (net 8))
 (segment (start 56.0363 81.1727) (end 56.8366 81.973) (width 0.25) (layer F.Cu) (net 8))
 (segment (start 56.8366 81.973) (end 56.8366 85.0811) (width 0.25) (layer F.Cu) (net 8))
 (segment (start 56.8366 85.0811) (end 56.1677 85.75) (width 0.25) (layer F.Cu) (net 8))
 (segment (start 56.1677 85.75) (end 55.5 85.75) (width 0.25) (layer F.Cu) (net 8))
 (segment (start 55.5 85.75) (end 55.5 88.25) (width 0.25) (layer F.Cu) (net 8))
 (segment (start 55.5 88.25) (end 55.75 88.5) (width 0.25) (layer F.Cu) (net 8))
 (segment (start 55.75 88.5) (end 55.8793 88.3707) (width 0.25) (layer F.Cu) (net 8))
 (segment (start 55.8793 88.3707) (end 59.15 88.3707) (width 0.25) (layer F.Cu) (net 8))
 (segment (start 57.865 66.675) (end 57.865 69.7953) (width 0.25) (layer F.Cu) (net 9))
 (segment (start 57.865 69.7953) (end 56.5 71.1603) (width 0.25) (layer F.Cu) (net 9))
 (segment (start 56.5 71.1603) (end 56.5 73) (width 0.25) (layer F.Cu) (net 9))
 (segment (start 56.5 73) (end 57.025 73.525) (width 0.25) (layer F.Cu) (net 9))
 (segment (start 57.025 73.525) (end 58.665 73.525) (width 0.25) (layer F.Cu) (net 9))
 (segment (start 51.6 64.8) (end 56.89 64.8) (width 0.25) (layer F.Cu) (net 9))
 (segment (start 56.89 64.8) (end 57.865 65.775) (width 0.25) (layer F.Cu) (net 9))
 (segment (start 57.865 65.775) (end 57.865 66.675) (width 0.25) (layer F.Cu) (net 9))
 (segment (start 57.865 66.675) (end 60.88 66.675) (width 0.25) (layer F.Cu) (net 9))
 (segment (start 60.98 64.135) (end 60.98 66.575) (width 0.25) (layer F.Cu) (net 9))
 (segment (start 60.98 66.575) (end 60.88 66.675) (width 0.25) (layer F.Cu) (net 9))
 (segment (start 61 69.5) (end 60.875 69.5) (width 0.25) (layer F.Cu) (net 11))
 (segment (start 60.875 69.5) (end 58.665 71.71) (width 0.25) (layer F.Cu) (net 11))
 (segment (start 58.665 71.71) (end 58.665 72.875) (width 0.25) (layer F.Cu) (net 11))
 (segment (start 81.6 69.6) (end 79.3499 69.6) (width 0.25) (layer F.Cu) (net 1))
 (segment (start 73.6 70.8) (end 78.1499 70.8) (width 0.25) (layer F.Cu) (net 1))
 (segment (start 78.1499 70.8) (end 79.3499 69.6) (width 0.25) (layer F.Cu) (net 1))
 (segment (start 72.7568 70.8) (end 73.6 70.8) (width 0.25) (layer F.Cu) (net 1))
 (segment (start 72.7568 70.8) (end 71.9135 70.8) (width 0.25) (layer F.Cu) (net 1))
 (segment (start 82.85 78) (end 82.85 77.0499) (width 0.25) (layer F.Cu) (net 1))
 (segment (start 82.85 77.0499) (end 79.9751 74.175) (width 0.25) (layer F.Cu) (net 1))
 (segment (start 79.9751 74.175) (end 65.8201 74.175) (width 0.25) (layer F.Cu) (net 1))
 (segment (start 71.9135 70.8) (end 70.2635 69.15) (width 0.25) (layer F.Cu) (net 1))
 (segment (start 70.2635 69.15) (end 67.4 69.15) (width 0.25) (layer F.Cu) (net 1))
 (segment (start 71.9135 70.8) (end 70.2269 70.8) (width 0.25) (layer F.Cu) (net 1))
 (segment (start 65.8201 73.525) (end 67.5019 73.525) (width 0.25) (layer F.Cu) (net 1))
 (segment (start 67.5019 73.525) (end 70.2269 70.8) (width 0.25) (layer F.Cu) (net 1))
 (segment (start 65.5715 74.175) (end 65.8201 73.9264) (width 0.25) (layer F.Cu) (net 1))
 (segment (start 65.8201 73.9264) (end 65.8201 73.525) (width 0.25) (layer F.Cu) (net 1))
 (segment (start 65.2126 74.175) (end 65.5715 74.175) (width 0.25) (layer F.Cu) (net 1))
 (segment (start 65.5715 74.175) (end 65.8201 74.175) (width 0.25) (layer F.Cu) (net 1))
 (segment (start 64.605 73.525) (end 65.8201 73.525) (width 0.25) (layer F.Cu) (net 1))
 (segment (start 64.605 74.175) (end 65.2126 74.175) (width 0.25) (layer F.Cu) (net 1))
 (segment (start 64.605 74.825) (end 65.8201 74.825) (width 0.25) (layer F.Cu) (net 1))
 (segment (start 65.8201 74.825) (end 65.8201 74.175) (width 0.25) (layer F.Cu) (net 1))
 (segment (start 64.605 72.875) (end 66.3 72.875) (width 0.25) (layer F.Cu) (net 12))
 (segment (start 66.3 72.875) (end 67.4 71.775) (width 0.25) (layer F.Cu) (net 12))
 (segment (start 67.4 71.775) (end 67.4 71.65) (width 0.25) (layer F.Cu) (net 12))
 (segment (start 75.886 77.15) (end 71.314 77.15) (width 0.25) (layer F.Cu) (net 14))
 (segment (start 65.8201 76.125) (end 69.1384 76.125) (width 0.25) (layer F.Cu) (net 14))
 (segment (start 69.1384 76.125) (end 70.1634 77.15) (width 0.25) (layer F.Cu) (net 14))
 (segment (start 71.314 77.15) (end 70.1634 77.15) (width 0.25) (layer F.Cu) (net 14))
 (segment (start 65.8201 76.125) (end 65.8201 75.475) (width 0.25) (layer F.Cu) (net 14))
 (segment (start 64.605 75.475) (end 65.8201 75.475) (width 0.25) (layer F.Cu) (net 14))
 (segment (start 64.605 76.125) (end 65.8201 76.125) (width 0.25) (layer F.Cu) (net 14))
 (segment (start 58.137 84.987) (end 58.637 84.987) (width 0.25) (layer F.Cu) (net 15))
 (segment (start 58.637 84.987) (end 59.15 85.5) (width 0.25) (layer F.Cu) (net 15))
 (segment (start 58.137 84.987) (end 58.65 85.5) (width 0.25) (layer F.Cu) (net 15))
 (segment (start 58.665 77.425) (end 57.525 77.425) (width 0.25) (layer F.Cu) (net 15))
 (segment (start 57.525 77.425) (end 56.5 78.45) (width 0.25) (layer F.Cu) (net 15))
 (segment (start 56.5 78.45) (end 56.5 80.6656) (width 0.25) (layer F.Cu) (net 15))
 (segment (start 56.5 80.6656) (end 57.624 81.7896) (width 0.25) (layer F.Cu) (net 15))
 (segment (start 57.624 81.7896) (end 57.624 84.474) (width 0.25) (layer F.Cu) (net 15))
 (segment (start 57.624 84.474) (end 58.137 84.987) (width 0.25) (layer F.Cu) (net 15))
 (segment (start 58.665 75.475) (end 53.925 75.475) (width 0.25) (layer F.Cu) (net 16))
 (segment (start 53.925 75.475) (end 52.8 76.6) (width 0.25) (layer F.Cu) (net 16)))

